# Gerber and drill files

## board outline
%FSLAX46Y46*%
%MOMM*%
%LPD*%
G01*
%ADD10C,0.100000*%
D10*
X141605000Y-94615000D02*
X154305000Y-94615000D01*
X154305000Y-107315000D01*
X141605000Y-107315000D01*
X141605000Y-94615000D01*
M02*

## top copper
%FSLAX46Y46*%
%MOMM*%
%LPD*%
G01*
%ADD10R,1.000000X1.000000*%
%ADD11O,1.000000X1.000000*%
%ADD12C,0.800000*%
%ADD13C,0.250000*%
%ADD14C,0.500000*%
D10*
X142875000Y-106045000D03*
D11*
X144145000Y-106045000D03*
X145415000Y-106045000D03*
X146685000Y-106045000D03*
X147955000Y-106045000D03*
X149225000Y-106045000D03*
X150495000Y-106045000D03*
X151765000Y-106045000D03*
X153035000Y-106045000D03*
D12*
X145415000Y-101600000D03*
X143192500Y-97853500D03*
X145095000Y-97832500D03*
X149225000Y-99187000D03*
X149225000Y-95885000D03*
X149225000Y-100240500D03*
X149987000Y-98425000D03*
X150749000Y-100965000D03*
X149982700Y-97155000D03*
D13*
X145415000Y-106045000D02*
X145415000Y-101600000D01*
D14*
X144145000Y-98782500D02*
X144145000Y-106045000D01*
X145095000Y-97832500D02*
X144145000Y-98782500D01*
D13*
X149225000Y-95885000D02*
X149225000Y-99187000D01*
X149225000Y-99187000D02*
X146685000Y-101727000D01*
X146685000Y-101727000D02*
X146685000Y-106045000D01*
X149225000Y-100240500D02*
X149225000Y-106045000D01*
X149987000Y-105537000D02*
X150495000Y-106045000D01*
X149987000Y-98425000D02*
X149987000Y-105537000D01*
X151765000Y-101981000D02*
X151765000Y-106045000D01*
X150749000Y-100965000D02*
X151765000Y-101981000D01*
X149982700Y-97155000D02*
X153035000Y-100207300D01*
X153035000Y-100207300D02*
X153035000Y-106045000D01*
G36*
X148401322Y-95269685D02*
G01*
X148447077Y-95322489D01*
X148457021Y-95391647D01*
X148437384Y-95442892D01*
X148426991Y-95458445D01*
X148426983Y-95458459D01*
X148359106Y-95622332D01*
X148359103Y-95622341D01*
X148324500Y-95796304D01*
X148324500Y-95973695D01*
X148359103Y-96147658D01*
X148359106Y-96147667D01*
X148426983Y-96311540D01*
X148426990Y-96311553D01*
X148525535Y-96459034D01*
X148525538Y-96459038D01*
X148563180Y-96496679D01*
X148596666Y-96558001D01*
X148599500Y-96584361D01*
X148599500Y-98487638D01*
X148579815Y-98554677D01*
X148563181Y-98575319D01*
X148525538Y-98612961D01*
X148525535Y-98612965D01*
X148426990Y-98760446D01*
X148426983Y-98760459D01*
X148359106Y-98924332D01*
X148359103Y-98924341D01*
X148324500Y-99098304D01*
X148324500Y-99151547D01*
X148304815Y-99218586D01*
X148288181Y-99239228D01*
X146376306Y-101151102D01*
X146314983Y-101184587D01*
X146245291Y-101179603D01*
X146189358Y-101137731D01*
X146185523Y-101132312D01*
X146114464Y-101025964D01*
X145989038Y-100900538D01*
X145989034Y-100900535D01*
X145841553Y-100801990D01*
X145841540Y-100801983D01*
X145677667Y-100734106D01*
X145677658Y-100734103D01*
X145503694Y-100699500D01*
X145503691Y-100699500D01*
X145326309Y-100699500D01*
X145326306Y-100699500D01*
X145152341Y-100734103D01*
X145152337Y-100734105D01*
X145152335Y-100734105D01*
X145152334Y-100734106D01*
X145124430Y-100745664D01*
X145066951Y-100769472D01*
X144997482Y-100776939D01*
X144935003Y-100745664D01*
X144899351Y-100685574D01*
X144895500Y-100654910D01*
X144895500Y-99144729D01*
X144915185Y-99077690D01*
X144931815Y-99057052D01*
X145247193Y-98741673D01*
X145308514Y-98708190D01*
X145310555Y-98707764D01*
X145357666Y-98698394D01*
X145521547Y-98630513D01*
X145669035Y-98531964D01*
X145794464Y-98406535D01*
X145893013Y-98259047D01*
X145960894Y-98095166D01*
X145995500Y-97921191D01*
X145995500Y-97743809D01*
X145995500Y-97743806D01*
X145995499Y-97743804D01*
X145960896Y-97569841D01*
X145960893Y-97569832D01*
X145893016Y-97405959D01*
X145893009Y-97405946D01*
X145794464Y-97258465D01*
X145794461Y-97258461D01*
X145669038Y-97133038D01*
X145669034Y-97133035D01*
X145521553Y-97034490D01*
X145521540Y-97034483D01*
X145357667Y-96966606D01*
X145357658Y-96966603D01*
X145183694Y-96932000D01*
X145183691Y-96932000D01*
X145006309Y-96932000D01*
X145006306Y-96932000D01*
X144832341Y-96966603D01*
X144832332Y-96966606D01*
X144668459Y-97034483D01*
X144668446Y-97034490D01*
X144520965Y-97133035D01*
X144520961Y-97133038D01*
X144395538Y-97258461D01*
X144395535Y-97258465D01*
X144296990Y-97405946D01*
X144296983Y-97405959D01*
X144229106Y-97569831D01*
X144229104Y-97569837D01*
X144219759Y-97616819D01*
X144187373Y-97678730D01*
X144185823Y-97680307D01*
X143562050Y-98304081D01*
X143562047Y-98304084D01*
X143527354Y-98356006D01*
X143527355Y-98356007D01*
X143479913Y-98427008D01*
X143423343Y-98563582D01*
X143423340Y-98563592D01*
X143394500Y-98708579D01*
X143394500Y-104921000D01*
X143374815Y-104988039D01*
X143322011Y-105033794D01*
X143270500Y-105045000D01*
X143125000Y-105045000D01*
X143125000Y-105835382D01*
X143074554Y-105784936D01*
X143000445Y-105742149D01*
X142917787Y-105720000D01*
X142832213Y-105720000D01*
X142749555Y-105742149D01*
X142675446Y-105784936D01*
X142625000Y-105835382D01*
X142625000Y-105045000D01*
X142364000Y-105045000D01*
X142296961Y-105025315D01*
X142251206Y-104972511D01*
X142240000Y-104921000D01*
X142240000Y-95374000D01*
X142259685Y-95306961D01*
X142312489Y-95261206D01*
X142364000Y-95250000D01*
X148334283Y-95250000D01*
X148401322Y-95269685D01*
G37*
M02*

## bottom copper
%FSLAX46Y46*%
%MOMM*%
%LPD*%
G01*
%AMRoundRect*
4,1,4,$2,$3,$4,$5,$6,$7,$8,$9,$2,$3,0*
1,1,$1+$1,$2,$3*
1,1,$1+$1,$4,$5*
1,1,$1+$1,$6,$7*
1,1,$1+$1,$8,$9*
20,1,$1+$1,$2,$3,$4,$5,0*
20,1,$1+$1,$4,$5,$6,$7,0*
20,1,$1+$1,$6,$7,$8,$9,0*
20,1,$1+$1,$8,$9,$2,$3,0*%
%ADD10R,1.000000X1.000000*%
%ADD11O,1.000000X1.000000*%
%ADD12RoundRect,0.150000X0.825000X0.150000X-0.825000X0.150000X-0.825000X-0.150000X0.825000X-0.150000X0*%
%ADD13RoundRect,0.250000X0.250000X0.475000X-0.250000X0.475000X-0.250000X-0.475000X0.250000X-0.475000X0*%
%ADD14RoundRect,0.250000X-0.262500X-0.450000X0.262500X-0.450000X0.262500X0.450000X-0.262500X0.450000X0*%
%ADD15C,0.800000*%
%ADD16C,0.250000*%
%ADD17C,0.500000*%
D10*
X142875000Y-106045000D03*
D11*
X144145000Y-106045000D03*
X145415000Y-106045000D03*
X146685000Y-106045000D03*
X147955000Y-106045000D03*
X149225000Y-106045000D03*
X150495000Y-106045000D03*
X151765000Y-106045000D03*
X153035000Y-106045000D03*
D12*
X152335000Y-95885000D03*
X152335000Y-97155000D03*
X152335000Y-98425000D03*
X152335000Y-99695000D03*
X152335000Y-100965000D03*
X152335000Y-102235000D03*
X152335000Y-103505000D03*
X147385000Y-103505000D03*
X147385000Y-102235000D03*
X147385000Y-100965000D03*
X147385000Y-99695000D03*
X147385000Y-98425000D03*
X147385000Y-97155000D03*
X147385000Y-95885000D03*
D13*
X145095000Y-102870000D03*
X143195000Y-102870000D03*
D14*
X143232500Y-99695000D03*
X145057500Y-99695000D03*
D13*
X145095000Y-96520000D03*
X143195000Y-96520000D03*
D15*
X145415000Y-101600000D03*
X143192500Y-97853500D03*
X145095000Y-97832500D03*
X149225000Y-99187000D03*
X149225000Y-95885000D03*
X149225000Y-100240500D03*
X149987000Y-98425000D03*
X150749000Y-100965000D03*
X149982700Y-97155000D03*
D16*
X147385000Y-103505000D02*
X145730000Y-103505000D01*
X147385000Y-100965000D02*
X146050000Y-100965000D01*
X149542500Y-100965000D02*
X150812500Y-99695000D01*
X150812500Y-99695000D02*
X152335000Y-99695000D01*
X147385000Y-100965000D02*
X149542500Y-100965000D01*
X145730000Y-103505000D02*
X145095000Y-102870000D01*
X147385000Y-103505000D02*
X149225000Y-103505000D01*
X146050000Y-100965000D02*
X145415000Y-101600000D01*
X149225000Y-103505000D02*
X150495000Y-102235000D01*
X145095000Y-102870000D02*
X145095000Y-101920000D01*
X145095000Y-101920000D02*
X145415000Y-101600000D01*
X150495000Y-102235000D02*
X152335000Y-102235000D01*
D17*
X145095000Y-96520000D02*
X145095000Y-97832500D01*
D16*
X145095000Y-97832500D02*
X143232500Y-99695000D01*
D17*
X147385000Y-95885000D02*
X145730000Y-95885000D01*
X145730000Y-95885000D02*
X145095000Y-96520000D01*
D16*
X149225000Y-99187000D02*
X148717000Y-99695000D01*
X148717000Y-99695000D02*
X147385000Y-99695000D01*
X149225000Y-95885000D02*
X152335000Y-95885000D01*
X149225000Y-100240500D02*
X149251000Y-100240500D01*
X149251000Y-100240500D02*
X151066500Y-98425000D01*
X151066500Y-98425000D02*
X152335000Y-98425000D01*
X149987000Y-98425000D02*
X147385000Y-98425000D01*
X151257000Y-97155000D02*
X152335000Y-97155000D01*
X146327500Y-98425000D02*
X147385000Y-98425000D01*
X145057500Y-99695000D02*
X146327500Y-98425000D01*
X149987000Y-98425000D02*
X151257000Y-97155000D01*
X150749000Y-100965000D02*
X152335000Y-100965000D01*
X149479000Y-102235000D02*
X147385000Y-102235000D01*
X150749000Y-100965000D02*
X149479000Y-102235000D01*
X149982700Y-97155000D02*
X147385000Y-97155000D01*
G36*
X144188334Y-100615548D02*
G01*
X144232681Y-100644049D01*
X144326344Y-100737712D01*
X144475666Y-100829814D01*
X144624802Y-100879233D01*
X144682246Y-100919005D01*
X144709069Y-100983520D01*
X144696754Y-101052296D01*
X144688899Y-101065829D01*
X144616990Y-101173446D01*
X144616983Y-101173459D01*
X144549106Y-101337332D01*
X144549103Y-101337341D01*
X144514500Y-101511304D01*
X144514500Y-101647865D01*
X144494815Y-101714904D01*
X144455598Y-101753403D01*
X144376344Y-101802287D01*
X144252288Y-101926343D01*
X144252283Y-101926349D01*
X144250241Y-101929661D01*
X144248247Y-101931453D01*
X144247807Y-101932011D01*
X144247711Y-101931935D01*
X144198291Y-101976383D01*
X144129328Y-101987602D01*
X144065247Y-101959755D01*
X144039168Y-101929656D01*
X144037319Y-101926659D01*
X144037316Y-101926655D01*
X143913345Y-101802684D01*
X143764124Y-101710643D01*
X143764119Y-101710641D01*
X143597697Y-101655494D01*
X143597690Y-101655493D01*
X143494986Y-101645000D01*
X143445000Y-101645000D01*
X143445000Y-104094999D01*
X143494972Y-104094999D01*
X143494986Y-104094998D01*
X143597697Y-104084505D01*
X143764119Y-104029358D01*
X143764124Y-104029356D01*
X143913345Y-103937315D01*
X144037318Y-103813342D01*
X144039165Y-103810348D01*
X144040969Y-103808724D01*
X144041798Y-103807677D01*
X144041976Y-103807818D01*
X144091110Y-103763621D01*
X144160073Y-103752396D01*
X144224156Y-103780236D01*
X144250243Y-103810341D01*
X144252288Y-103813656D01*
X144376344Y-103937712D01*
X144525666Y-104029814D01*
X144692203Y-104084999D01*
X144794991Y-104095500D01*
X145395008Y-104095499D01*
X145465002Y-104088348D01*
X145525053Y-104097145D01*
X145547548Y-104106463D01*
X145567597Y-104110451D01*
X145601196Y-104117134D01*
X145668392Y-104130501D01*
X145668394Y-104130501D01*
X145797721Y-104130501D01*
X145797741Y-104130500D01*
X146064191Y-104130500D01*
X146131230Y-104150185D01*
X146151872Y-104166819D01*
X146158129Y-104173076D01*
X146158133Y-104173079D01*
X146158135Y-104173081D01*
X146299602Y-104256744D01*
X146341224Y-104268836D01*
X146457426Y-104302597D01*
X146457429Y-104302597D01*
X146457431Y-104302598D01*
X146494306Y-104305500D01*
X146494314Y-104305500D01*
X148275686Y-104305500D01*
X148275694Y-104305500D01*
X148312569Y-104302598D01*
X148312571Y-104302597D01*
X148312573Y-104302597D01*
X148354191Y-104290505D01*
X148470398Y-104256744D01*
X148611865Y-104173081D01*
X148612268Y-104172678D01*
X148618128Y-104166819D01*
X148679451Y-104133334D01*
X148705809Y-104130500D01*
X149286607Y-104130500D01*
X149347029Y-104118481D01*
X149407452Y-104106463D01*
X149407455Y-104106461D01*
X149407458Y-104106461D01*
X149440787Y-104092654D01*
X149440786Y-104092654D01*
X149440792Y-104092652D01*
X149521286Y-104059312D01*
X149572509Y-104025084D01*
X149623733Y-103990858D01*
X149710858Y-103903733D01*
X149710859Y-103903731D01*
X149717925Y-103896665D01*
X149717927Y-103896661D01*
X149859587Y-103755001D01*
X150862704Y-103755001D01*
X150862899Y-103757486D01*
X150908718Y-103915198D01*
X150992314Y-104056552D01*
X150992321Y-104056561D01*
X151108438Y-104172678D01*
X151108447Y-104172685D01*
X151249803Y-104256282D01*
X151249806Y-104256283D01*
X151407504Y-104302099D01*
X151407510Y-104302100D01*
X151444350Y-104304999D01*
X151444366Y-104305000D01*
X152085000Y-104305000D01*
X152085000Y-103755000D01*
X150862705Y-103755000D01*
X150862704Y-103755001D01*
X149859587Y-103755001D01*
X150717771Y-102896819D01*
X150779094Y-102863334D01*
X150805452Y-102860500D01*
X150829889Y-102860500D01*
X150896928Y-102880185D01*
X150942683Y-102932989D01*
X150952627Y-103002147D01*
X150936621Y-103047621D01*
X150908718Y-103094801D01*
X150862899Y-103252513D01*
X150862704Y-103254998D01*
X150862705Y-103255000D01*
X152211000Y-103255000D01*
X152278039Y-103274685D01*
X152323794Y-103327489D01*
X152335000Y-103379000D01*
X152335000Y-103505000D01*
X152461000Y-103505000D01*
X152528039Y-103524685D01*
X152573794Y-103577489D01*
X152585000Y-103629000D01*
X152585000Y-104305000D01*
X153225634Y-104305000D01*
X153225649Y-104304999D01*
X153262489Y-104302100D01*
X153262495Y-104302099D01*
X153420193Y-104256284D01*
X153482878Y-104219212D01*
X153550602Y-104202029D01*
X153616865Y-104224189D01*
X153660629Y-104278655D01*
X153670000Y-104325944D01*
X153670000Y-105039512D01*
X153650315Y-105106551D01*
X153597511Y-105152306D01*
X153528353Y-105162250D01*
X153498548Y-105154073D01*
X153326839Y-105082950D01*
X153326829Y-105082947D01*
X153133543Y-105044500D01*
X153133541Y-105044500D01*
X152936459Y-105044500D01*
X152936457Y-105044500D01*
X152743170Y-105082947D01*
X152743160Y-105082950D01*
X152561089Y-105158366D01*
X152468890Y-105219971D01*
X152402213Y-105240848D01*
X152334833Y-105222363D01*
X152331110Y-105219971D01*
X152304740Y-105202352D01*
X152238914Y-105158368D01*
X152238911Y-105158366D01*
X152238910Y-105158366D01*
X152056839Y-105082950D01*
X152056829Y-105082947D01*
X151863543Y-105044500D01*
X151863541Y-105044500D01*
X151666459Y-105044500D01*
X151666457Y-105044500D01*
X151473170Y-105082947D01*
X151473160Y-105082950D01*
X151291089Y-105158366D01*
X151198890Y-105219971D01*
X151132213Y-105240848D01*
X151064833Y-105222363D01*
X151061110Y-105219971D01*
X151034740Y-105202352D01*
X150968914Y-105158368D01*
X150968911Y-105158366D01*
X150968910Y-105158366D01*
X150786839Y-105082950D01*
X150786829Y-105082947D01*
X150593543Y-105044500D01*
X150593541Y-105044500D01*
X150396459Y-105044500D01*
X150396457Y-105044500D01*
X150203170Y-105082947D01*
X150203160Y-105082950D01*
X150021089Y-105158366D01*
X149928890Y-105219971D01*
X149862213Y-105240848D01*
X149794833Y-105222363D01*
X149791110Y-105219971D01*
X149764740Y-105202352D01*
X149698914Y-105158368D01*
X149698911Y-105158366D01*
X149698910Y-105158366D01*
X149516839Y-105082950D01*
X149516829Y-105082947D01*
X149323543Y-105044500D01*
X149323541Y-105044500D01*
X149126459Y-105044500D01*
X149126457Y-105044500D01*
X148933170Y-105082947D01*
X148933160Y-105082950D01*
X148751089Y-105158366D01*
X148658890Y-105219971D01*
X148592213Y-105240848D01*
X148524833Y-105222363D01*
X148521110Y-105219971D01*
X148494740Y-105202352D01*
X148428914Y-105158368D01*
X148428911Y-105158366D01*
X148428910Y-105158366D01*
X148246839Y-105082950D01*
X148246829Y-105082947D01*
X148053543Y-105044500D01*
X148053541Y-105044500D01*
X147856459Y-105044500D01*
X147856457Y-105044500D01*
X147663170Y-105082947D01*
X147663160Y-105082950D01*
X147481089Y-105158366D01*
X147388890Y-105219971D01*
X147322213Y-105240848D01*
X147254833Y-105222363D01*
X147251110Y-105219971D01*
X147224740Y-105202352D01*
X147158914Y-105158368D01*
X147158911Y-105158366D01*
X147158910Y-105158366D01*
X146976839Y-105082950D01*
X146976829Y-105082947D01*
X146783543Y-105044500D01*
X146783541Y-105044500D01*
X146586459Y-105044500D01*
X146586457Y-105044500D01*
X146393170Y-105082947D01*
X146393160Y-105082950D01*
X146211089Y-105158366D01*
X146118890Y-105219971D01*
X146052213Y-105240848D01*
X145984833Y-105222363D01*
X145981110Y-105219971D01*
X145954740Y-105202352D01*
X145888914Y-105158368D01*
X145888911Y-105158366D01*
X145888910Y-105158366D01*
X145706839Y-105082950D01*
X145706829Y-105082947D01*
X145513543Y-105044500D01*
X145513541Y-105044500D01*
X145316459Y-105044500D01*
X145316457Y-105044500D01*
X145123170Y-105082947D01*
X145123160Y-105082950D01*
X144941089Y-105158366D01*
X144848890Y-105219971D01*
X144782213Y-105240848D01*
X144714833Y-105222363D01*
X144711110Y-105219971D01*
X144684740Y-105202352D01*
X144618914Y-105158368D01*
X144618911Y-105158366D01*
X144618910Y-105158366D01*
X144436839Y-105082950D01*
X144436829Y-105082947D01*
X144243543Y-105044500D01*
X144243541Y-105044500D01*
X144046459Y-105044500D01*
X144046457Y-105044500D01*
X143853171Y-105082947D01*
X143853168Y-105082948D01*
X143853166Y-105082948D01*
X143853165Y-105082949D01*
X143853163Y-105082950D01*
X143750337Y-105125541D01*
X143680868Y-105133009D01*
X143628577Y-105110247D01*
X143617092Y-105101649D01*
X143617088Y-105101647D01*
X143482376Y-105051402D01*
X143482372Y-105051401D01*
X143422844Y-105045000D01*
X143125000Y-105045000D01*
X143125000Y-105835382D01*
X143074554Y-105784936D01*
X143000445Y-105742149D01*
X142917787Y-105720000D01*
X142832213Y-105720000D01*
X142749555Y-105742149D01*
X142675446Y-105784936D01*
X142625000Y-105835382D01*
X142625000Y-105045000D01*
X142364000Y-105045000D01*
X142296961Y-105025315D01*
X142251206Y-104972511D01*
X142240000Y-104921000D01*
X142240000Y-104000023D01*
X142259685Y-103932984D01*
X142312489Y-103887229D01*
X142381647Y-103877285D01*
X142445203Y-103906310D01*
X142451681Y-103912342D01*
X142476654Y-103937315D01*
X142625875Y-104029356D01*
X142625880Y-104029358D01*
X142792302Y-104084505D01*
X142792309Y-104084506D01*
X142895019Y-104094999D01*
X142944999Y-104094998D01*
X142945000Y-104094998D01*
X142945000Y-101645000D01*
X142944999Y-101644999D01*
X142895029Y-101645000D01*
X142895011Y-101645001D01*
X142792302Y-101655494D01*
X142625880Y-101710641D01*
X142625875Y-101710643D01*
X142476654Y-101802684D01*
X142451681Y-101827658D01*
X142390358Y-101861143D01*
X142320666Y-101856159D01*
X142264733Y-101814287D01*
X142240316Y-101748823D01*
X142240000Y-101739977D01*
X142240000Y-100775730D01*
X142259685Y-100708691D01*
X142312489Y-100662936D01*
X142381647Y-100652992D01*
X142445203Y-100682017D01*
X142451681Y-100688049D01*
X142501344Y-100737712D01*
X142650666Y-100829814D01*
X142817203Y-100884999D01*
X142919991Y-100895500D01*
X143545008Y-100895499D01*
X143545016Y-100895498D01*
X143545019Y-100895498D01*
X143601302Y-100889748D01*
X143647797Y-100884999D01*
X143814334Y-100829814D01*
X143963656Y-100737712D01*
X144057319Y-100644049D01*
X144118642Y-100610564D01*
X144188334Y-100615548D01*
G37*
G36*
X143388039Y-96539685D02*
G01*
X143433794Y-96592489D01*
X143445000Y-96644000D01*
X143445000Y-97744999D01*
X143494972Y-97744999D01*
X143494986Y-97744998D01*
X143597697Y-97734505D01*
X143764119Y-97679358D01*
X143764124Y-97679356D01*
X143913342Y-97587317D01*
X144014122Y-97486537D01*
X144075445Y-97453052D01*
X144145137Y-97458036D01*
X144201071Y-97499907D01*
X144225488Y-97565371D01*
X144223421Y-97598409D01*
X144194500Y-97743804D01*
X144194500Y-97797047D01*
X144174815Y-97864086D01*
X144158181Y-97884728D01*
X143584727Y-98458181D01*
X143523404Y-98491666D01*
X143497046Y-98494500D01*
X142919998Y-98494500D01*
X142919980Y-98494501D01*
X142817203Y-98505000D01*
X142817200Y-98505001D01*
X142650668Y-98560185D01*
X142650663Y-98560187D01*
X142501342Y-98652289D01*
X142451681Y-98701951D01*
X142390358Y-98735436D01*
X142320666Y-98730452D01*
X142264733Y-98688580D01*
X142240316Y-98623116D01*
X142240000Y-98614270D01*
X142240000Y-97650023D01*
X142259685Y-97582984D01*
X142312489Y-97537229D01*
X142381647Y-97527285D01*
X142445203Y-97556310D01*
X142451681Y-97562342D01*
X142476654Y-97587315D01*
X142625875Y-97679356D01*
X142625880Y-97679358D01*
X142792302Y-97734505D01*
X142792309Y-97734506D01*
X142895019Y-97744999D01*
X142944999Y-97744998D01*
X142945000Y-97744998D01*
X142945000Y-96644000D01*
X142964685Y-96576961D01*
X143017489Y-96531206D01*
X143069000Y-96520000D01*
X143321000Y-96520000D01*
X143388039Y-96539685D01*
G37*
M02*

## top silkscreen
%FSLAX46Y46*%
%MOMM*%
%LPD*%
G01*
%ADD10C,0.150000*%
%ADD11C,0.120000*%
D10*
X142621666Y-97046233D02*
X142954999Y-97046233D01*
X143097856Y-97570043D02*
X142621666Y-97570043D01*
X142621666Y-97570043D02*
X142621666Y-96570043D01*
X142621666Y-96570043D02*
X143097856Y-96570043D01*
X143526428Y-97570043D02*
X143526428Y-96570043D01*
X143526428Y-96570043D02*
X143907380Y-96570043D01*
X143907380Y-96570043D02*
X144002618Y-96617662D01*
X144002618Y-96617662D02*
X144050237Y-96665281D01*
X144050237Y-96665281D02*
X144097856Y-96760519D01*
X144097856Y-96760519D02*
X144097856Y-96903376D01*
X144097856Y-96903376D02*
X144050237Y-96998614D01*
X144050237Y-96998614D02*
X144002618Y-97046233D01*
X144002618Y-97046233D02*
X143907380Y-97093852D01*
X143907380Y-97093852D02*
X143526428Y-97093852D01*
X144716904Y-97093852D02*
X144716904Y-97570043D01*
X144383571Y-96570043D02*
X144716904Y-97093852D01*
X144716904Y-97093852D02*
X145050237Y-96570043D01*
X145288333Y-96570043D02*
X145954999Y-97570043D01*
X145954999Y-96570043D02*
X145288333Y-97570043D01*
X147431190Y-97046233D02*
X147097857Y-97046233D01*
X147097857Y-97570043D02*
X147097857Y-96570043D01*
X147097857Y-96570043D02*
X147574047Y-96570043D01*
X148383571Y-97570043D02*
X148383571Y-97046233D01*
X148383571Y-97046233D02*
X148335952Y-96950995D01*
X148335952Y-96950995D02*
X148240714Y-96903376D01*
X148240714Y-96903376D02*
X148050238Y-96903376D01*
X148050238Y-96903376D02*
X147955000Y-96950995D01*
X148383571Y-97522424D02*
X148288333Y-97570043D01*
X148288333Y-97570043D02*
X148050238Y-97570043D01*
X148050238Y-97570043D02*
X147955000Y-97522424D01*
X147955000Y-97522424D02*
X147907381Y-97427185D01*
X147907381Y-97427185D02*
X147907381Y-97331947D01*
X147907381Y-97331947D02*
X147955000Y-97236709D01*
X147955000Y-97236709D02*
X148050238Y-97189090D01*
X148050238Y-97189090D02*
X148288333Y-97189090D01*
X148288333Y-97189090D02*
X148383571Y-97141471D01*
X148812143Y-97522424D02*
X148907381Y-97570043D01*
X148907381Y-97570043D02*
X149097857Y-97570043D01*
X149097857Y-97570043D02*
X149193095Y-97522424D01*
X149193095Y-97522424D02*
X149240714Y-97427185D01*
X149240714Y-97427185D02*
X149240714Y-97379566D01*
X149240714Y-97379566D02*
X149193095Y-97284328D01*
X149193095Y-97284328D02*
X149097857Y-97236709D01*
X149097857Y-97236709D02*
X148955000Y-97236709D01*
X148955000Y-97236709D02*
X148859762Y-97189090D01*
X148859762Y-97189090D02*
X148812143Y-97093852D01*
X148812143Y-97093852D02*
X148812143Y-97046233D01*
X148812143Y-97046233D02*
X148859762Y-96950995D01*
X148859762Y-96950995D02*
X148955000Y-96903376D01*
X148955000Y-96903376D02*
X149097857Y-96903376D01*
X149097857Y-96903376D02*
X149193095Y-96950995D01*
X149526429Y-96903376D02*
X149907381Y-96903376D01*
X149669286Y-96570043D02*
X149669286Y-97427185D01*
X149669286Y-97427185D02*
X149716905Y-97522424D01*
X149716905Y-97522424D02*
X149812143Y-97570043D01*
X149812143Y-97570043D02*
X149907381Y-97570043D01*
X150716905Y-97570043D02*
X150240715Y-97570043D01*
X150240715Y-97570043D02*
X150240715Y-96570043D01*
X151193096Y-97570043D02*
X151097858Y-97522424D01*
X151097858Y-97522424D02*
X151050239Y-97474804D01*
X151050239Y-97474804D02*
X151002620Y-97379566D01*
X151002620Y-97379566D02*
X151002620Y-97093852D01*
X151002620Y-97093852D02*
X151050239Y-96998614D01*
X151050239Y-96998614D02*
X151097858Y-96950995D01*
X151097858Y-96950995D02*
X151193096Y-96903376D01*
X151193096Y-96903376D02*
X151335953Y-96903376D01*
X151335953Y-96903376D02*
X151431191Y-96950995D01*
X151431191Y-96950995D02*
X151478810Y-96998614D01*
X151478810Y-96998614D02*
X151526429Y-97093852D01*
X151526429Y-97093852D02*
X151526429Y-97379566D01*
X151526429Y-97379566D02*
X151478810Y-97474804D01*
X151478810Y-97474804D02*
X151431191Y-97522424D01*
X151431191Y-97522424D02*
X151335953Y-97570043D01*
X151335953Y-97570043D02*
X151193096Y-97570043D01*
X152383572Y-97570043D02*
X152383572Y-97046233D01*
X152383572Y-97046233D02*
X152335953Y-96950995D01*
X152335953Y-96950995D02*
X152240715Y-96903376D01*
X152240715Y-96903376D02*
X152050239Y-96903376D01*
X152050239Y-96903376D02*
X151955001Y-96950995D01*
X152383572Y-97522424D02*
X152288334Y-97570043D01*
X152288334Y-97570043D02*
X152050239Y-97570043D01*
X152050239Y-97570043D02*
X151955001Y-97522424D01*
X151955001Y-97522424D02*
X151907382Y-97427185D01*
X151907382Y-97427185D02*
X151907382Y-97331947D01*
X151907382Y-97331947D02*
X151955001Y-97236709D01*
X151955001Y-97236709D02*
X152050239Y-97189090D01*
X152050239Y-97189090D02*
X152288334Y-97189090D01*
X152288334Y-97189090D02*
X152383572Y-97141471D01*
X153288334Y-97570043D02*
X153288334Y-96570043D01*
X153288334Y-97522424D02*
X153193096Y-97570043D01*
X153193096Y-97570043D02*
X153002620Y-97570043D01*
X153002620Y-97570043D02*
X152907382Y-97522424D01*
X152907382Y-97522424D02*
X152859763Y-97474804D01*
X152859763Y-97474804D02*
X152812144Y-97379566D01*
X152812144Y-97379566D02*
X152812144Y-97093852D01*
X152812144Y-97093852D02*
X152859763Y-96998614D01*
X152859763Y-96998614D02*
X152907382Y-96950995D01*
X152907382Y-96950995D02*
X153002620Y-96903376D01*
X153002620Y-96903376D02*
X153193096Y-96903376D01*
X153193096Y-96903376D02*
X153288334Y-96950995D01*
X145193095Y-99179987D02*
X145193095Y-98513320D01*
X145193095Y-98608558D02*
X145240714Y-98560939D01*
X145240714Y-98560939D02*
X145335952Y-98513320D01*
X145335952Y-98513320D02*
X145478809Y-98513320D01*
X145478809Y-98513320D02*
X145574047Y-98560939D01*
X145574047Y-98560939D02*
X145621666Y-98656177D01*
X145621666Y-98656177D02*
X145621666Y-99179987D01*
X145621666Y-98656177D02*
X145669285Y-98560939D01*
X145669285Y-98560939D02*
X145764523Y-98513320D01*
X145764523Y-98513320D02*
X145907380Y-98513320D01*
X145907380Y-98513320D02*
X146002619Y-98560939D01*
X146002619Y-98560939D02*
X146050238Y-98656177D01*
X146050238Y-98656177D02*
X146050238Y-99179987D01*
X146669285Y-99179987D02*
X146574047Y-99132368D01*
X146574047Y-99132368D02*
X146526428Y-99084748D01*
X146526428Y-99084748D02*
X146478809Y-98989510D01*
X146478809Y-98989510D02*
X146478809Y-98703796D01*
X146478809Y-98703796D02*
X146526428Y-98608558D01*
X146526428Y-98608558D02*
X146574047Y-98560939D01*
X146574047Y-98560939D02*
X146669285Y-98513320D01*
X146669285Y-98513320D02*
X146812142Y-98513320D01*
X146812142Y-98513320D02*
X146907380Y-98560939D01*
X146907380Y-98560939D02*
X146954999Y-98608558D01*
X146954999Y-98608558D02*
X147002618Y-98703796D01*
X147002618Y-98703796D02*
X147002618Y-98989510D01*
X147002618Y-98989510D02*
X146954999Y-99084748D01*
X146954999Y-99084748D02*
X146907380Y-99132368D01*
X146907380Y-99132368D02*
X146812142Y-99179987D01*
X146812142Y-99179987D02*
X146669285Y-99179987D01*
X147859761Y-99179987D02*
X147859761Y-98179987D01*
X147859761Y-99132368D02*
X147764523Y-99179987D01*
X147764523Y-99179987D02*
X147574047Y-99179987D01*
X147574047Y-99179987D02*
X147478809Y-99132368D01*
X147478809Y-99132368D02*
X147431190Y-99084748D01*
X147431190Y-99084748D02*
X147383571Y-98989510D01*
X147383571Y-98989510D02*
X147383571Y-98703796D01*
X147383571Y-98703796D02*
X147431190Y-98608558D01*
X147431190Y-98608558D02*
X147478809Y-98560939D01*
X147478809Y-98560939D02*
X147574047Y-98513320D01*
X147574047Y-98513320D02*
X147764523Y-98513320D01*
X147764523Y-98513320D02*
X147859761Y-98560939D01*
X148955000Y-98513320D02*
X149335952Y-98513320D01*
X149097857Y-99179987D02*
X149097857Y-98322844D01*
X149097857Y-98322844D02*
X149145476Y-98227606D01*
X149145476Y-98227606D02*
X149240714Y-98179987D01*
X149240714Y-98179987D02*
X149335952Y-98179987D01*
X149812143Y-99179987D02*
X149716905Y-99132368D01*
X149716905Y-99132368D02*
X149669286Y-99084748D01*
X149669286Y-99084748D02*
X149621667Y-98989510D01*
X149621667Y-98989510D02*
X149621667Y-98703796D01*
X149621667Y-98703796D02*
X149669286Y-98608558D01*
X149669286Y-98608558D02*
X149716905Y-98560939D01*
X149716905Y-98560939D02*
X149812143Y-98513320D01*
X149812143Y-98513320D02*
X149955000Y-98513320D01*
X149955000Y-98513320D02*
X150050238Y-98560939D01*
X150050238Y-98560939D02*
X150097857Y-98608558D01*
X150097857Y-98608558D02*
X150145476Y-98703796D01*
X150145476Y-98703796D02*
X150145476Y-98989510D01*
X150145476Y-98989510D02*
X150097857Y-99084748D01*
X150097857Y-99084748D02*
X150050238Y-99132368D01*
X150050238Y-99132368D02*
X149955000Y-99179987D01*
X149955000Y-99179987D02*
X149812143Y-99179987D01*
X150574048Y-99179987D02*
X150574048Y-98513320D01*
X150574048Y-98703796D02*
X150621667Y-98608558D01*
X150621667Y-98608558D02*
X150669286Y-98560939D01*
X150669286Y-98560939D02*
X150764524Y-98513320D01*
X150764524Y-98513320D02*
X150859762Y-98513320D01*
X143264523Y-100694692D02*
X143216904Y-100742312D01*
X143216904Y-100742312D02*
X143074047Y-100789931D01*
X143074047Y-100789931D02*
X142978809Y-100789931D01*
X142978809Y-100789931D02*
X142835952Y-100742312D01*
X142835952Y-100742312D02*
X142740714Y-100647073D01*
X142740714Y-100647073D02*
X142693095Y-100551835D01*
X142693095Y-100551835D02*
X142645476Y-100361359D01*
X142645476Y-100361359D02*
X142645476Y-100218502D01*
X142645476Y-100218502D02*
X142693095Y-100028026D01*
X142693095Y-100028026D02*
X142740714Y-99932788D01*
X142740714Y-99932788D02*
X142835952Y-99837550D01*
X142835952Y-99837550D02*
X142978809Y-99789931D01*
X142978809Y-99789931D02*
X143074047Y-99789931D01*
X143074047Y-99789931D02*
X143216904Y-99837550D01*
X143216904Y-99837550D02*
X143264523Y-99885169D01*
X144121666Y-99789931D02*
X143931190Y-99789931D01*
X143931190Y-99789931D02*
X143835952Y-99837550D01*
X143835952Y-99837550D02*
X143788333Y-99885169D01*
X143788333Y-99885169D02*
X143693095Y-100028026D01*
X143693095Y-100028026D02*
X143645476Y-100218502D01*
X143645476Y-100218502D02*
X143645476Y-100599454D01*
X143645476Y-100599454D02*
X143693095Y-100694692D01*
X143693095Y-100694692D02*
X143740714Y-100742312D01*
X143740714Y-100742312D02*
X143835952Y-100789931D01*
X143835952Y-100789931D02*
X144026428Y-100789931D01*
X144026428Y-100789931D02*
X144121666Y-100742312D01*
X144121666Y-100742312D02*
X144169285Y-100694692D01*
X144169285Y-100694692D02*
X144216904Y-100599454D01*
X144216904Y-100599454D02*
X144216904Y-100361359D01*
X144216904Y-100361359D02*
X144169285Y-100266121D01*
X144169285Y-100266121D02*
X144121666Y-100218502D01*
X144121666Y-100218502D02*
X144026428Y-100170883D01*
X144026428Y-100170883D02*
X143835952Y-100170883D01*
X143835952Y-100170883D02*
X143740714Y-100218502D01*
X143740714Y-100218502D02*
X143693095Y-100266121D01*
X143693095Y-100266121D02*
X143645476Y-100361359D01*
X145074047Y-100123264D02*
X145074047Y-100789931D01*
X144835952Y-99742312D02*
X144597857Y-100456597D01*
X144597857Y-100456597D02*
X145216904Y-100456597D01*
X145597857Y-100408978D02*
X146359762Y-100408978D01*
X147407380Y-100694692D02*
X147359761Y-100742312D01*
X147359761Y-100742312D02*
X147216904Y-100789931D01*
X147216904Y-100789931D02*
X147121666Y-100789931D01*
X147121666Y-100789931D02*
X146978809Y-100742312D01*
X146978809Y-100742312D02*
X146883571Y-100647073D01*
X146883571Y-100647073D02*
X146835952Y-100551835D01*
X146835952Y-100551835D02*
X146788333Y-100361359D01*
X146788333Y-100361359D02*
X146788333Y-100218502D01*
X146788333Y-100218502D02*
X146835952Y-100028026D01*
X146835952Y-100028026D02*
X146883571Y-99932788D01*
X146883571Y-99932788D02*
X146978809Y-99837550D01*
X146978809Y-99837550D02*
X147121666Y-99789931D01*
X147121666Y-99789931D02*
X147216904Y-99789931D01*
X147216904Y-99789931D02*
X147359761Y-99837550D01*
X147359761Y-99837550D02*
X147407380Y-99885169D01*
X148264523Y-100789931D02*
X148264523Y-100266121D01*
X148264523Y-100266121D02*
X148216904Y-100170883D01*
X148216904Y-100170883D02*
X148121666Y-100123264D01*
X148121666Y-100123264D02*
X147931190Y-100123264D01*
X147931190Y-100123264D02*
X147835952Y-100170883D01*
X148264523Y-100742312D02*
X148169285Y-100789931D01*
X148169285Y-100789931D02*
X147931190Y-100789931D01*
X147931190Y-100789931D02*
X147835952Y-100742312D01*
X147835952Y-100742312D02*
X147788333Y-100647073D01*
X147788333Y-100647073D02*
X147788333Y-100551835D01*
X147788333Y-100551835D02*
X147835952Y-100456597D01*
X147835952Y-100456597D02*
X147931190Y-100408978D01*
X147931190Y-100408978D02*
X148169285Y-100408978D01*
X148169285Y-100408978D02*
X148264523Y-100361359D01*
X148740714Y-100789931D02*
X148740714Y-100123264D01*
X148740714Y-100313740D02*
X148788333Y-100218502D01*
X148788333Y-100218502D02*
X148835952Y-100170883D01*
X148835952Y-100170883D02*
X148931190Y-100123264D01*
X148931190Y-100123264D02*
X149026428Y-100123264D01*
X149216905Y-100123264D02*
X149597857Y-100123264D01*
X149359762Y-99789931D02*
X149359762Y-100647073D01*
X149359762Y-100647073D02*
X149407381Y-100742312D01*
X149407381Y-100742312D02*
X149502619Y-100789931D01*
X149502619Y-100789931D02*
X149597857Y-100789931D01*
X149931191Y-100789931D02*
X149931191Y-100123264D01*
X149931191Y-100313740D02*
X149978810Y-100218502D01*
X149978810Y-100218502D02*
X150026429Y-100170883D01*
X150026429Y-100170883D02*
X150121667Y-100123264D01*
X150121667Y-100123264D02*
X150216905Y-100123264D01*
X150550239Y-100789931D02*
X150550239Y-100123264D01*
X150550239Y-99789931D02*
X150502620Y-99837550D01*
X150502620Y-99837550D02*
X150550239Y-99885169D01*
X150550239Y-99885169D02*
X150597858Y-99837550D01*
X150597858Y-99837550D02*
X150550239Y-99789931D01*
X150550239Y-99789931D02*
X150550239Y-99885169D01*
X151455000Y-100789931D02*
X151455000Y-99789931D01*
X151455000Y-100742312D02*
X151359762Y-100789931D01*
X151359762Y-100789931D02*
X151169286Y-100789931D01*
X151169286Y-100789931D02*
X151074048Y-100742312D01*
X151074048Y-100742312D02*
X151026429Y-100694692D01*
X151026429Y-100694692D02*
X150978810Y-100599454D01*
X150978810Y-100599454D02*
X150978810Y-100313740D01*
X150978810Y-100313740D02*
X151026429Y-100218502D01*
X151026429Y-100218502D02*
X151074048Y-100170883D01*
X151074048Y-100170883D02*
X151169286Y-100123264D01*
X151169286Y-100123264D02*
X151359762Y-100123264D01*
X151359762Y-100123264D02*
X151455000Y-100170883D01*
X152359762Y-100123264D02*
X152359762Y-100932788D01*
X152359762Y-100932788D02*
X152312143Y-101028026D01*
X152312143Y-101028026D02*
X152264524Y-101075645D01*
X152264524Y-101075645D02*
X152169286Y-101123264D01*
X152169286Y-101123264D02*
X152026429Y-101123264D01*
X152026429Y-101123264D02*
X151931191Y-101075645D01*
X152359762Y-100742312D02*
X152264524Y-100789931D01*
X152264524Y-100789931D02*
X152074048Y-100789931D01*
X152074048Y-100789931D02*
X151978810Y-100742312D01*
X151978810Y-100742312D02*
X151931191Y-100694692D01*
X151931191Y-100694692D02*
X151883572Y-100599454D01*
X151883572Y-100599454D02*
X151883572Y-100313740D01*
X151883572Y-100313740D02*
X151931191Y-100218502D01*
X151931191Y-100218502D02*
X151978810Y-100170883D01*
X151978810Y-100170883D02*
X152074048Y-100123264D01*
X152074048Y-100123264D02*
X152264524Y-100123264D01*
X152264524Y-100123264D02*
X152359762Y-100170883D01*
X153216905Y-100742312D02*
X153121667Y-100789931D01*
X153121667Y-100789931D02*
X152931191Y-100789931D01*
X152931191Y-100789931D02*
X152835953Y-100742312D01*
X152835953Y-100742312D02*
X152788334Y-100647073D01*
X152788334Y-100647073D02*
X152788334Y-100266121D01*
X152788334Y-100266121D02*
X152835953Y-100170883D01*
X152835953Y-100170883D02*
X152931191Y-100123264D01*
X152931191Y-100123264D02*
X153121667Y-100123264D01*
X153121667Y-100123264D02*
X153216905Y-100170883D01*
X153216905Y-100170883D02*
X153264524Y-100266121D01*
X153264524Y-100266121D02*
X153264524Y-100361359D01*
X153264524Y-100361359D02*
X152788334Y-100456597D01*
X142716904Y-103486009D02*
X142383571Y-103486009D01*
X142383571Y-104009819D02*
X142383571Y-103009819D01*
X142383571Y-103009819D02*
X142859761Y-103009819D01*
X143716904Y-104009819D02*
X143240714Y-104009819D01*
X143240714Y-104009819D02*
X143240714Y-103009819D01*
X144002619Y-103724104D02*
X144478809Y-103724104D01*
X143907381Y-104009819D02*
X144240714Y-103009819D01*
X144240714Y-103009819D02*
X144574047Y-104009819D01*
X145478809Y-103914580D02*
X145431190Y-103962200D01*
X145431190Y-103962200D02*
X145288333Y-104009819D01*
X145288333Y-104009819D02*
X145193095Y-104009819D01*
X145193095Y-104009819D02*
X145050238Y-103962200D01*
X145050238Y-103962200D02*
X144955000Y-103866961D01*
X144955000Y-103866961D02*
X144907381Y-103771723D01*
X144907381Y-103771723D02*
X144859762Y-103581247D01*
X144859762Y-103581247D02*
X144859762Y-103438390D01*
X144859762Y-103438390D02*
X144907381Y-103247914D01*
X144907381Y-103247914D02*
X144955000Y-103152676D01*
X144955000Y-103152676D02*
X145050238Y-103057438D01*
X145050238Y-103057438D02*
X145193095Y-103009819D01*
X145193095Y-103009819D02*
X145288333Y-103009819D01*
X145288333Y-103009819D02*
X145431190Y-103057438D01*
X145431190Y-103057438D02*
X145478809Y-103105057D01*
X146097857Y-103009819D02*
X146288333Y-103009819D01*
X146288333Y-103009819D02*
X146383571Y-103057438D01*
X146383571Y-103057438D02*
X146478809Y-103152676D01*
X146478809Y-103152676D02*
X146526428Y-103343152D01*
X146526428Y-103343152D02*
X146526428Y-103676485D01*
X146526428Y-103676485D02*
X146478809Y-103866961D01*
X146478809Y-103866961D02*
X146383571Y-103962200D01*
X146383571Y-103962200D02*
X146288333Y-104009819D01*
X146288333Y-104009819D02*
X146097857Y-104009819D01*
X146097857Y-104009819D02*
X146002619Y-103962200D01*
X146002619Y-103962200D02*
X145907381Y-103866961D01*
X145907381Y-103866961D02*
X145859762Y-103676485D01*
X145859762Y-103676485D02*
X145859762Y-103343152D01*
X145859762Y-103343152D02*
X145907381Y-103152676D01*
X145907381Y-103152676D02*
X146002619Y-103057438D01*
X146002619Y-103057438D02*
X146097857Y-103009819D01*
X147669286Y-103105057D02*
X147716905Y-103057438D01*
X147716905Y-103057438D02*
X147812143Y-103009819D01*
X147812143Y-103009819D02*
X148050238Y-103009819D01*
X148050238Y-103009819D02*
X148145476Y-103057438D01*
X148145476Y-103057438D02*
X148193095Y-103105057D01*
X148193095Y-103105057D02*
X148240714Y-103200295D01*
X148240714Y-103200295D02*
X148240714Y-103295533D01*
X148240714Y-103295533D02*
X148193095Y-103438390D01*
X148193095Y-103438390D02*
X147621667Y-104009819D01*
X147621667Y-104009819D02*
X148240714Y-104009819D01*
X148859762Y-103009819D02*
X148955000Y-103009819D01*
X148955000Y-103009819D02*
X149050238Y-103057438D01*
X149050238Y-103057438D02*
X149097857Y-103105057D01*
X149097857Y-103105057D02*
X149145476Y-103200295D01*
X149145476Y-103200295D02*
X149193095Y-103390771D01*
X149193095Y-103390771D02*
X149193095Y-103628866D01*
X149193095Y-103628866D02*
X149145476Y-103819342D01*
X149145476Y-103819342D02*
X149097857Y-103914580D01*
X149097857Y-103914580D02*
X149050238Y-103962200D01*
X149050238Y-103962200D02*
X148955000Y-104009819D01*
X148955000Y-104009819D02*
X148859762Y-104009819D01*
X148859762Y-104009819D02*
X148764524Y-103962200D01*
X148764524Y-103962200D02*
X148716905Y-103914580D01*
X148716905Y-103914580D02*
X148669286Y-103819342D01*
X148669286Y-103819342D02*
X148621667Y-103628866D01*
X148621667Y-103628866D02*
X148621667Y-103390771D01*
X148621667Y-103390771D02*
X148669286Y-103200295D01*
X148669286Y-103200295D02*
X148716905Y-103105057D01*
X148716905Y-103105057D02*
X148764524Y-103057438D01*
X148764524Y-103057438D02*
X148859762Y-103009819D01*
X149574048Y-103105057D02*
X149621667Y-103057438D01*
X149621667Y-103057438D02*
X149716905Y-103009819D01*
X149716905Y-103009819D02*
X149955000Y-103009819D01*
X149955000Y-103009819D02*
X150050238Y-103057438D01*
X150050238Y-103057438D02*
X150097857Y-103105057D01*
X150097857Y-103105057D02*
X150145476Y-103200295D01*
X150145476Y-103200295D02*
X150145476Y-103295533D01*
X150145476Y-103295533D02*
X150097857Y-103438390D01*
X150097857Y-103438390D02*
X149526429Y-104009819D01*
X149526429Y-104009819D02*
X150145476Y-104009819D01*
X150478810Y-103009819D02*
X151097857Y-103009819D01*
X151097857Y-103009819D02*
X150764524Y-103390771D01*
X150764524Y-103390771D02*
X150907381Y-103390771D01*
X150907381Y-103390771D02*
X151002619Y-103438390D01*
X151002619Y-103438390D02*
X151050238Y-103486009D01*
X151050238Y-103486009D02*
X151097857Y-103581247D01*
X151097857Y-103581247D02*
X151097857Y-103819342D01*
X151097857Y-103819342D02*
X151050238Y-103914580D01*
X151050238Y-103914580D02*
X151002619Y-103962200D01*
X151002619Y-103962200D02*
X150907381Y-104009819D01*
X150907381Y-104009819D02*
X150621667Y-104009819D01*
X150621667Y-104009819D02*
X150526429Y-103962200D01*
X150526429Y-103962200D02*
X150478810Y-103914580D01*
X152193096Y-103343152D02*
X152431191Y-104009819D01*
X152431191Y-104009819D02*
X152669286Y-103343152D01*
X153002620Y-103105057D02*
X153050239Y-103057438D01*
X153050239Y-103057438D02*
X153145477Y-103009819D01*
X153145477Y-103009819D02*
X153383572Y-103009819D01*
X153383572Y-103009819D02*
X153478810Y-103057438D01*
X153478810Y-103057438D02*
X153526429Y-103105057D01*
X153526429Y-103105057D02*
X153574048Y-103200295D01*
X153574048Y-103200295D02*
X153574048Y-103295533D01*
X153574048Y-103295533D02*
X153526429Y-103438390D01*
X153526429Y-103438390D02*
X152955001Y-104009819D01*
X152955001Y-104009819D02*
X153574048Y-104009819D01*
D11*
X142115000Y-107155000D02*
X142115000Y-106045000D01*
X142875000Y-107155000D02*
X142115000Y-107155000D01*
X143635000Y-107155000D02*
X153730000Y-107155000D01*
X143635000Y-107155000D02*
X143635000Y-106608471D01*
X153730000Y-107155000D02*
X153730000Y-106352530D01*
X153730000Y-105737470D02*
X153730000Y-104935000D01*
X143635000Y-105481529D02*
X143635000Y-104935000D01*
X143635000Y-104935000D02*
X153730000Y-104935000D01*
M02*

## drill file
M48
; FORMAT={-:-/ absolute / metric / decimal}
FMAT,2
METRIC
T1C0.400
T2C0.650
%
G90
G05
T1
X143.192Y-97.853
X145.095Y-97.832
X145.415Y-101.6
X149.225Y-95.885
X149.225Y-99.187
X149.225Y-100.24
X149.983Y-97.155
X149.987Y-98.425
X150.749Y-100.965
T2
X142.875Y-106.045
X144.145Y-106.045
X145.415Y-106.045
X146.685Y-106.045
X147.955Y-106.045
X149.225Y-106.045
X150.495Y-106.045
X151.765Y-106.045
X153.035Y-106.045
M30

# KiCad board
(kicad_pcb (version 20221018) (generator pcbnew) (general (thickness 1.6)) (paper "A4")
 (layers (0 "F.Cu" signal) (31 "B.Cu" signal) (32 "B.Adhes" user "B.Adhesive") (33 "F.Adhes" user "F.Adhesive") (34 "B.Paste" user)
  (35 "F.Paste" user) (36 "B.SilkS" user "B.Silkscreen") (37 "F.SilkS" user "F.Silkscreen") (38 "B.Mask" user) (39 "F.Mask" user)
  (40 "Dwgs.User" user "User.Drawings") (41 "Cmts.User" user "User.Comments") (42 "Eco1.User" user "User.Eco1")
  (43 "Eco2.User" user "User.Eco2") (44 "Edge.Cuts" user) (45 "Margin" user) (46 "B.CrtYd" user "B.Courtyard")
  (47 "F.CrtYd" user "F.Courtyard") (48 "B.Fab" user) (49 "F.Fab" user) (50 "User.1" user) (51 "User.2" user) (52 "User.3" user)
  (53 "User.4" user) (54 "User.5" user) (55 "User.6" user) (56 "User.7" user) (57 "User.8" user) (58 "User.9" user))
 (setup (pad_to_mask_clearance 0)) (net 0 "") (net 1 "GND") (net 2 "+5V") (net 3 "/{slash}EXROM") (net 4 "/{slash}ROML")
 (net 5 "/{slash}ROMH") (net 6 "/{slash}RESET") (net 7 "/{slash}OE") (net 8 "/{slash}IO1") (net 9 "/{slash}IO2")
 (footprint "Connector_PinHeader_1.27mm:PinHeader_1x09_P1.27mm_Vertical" (layer "F.Cu") (at 142.875 106.045 90)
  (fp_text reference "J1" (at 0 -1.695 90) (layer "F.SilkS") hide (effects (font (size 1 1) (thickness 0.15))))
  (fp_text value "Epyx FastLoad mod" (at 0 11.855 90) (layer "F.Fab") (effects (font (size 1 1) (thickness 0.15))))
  (fp_line (start -1.11 -0.76) (end 0 -0.76) (stroke (width 0.12) (type solid)) (layer "F.SilkS"))
  (fp_line (start -1.11 0) (end -1.11 -0.76) (stroke (width 0.12) (type solid)) (layer "F.SilkS"))
  (fp_line (start -1.11 0.76) (end -1.11 10.855) (stroke (width 0.12) (type solid)) (layer "F.SilkS"))
  (fp_line (start -1.11 0.76) (end -0.563471 0.76) (stroke (width 0.12) (type solid)) (layer "F.SilkS"))
  (fp_line (start -1.11 10.855) (end -0.30753 10.855) (stroke (width 0.12) (type solid)) (layer "F.SilkS"))
  (fp_line (start 0.30753 10.855) (end 1.11 10.855) (stroke (width 0.12) (type solid)) (layer "F.SilkS"))
  (fp_line (start 0.563471 0.76) (end 1.11 0.76) (stroke (width 0.12) (type solid)) (layer "F.SilkS"))
  (fp_line (start 1.11 0.76) (end 1.11 10.855) (stroke (width 0.12) (type solid)) (layer "F.SilkS"))
  (pad "1" thru_hole rect (at 0 0 90) (size 1 1) (drill 0.65) (layers "*.Cu" "*.Mask") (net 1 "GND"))
  (pad "2" thru_hole oval (at 0 1.27 90) (size 1 1) (drill 0.65) (layers "*.Cu" "*.Mask") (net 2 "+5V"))
  (pad "3" thru_hole oval (at 0 2.54 90) (size 1 1) (drill 0.65) (layers "*.Cu" "*.Mask") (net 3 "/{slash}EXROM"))
  (pad "4" thru_hole oval (at 0 3.81 90) (size 1 1) (drill 0.65) (layers "*.Cu" "*.Mask") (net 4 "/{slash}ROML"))
  (pad "5" thru_hole oval (at 0 5.08 90) (size 1 1) (drill 0.65) (layers "*.Cu" "*.Mask") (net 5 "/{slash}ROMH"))
  (pad "6" thru_hole oval (at 0 6.35 90) (size 1 1) (drill 0.65) (layers "*.Cu" "*.Mask") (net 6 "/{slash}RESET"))
  (pad "7" thru_hole oval (at 0 7.62 90) (size 1 1) (drill 0.65) (layers "*.Cu" "*.Mask") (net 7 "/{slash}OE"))
  (pad "8" thru_hole oval (at 0 8.89 90) (size 1 1) (drill 0.65) (layers "*.Cu" "*.Mask") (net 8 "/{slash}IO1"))
  (pad "9" thru_hole oval (at 0 10.16 90) (size 1 1) (drill 0.65) (layers "*.Cu" "*.Mask") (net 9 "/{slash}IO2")))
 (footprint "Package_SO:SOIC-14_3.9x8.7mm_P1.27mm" (layer "B.Cu") (at 149.86 99.695 180)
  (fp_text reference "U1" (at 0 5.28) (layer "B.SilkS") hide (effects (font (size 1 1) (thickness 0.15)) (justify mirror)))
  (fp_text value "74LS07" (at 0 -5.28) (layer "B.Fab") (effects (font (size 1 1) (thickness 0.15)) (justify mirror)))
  (pad "1" smd roundrect (at -2.475 3.81 180) (size 1.95 0.6) (layers "B.Cu" "B.Paste" "B.Mask") (roundrect_rratio 0.25)
   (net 4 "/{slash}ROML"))
  (pad "2" smd roundrect (at -2.475 2.54 180) (size 1.95 0.6) (layers "B.Cu" "B.Paste" "B.Mask") (roundrect_rratio 0.25)
   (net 7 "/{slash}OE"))
  (pad "3" smd roundrect (at -2.475 1.27 180) (size 1.95 0.6) (layers "B.Cu" "B.Paste" "B.Mask") (roundrect_rratio 0.25)
   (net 6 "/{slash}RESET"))
  (pad "4" smd roundrect (at -2.475 0 180) (size 1.95 0.6) (layers "B.Cu" "B.Paste" "B.Mask") (roundrect_rratio 0.25)
   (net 3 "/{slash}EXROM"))
  (pad "5" smd roundrect (at -2.475 -1.27 180) (size 1.95 0.6) (layers "B.Cu" "B.Paste" "B.Mask") (roundrect_rratio 0.25)
   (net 8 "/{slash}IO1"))
  (pad "6" smd roundrect (at -2.475 -2.54 180) (size 1.95 0.6) (layers "B.Cu" "B.Paste" "B.Mask") (roundrect_rratio 0.25)
   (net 3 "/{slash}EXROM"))
  (pad "7" smd roundrect (at -2.475 -3.81 180) (size 1.95 0.6) (layers "B.Cu" "B.Paste" "B.Mask") (roundrect_rratio 0.25) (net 1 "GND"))
  (pad "8" smd roundrect (at 2.475 -3.81 180) (size 1.95 0.6) (layers "B.Cu" "B.Paste" "B.Mask") (roundrect_rratio 0.25)
   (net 3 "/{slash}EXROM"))
  (pad "9" smd roundrect (at 2.475 -2.54 180) (size 1.95 0.6) (layers "B.Cu" "B.Paste" "B.Mask") (roundrect_rratio 0.25)
   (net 8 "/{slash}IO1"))
  (pad "10" smd roundrect (at 2.475 -1.27 180) (size 1.95 0.6) (layers "B.Cu" "B.Paste" "B.Mask") (roundrect_rratio 0.25)
   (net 3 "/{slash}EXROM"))
  (pad "11" smd roundrect (at 2.475 0 180) (size 1.95 0.6) (layers "B.Cu" "B.Paste" "B.Mask") (roundrect_rratio 0.25) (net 4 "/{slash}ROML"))
  (pad "12" smd roundrect (at 2.475 1.27 180) (size 1.95 0.6) (layers "B.Cu" "B.Paste" "B.Mask") (roundrect_rratio 0.25)
   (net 7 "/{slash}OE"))
  (pad "13" smd roundrect (at 2.475 2.54 180) (size 1.95 0.6) (layers "B.Cu" "B.Paste" "B.Mask") (roundrect_rratio 0.25)
   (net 9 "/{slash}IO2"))
  (pad "14" smd roundrect (at 2.475 3.81 180) (size 1.95 0.6) (layers "B.Cu" "B.Paste" "B.Mask") (roundrect_rratio 0.25) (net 2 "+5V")))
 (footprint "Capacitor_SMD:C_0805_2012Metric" (layer "B.Cu") (at 144.145 102.87 180)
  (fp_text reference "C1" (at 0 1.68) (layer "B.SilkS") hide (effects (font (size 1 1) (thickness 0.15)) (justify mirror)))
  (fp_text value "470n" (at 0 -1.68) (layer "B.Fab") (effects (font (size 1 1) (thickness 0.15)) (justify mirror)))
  (pad "1" smd roundrect (at -0.95 0 180) (size 1 1.45) (layers "B.Cu" "B.Paste" "B.Mask") (roundrect_rratio 0.25) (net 3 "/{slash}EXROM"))
  (pad "2" smd roundrect (at 0.95 0 180) (size 1 1.45) (layers "B.Cu" "B.Paste" "B.Mask") (roundrect_rratio 0.25) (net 1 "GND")))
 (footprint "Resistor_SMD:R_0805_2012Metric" (layer "B.Cu") (at 144.145 99.695)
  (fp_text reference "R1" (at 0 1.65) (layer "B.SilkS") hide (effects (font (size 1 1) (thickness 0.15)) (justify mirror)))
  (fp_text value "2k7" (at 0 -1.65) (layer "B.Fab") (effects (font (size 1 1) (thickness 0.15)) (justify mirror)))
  (pad "1" smd roundrect (at -0.9125 0) (size 1.025 1.4) (layers "B.Cu" "B.Paste" "B.Mask") (roundrect_rratio 0.243902) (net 2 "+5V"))
  (pad "2" smd roundrect (at 0.9125 0) (size 1.025 1.4) (layers "B.Cu" "B.Paste" "B.Mask") (roundrect_rratio 0.243902) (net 7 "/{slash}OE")))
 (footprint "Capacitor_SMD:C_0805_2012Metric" (layer "B.Cu") (at 144.145 96.52 180)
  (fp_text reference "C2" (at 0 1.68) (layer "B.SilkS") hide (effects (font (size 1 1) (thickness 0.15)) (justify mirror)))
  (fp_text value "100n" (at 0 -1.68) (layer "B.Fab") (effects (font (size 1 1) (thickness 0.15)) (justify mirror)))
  (pad "1" smd roundrect (at -0.95 0 180) (size 1 1.45) (layers "B.Cu" "B.Paste" "B.Mask") (roundrect_rratio 0.25) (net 2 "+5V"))
  (pad "2" smd roundrect (at 0.95 0 180) (size 1 1.45) (layers "B.Cu" "B.Paste" "B.Mask") (roundrect_rratio 0.25) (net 1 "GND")))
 (gr_rect (start 141.605 94.615) (end 154.305 107.315) (stroke (width 0.1) (type default)) (fill none) (layer "Edge.Cuts"))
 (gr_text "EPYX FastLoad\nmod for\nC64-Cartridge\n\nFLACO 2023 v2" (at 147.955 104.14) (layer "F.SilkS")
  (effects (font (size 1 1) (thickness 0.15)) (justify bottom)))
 (segment (start 145.415 106.045) (end 145.415 101.6) (width 0.25) (layer "F.Cu") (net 3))
 (via (at 145.415 101.6) (size 0.8) (drill 0.4) (layers "F.Cu" "B.Cu") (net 3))
 (segment (start 147.385 103.505) (end 145.73 103.505) (width 0.25) (layer "B.Cu") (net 3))
 (segment (start 147.385 100.965) (end 146.05 100.965) (width 0.25) (layer "B.Cu") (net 3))
 (segment (start 149.5425 100.965) (end 150.8125 99.695) (width 0.25) (layer "B.Cu") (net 3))
 (segment (start 150.8125 99.695) (end 152.335 99.695) (width 0.25) (layer "B.Cu") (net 3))
 (segment (start 147.385 100.965) (end 149.5425 100.965) (width 0.25) (layer "B.Cu") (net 3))
 (segment (start 145.73 103.505) (end 145.095 102.87) (width 0.25) (layer "B.Cu") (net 3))
 (segment (start 147.385 103.505) (end 149.225 103.505) (width 0.25) (layer "B.Cu") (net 3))
 (segment (start 146.05 100.965) (end 145.415 101.6) (width 0.25) (layer "B.Cu") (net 3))
 (segment (start 149.225 103.505) (end 150.495 102.235) (width 0.25) (layer "B.Cu") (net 3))
 (segment (start 145.095 102.87) (end 145.095 101.92) (width 0.25) (layer "B.Cu") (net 3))
 (segment (start 145.095 101.92) (end 145.415 101.6) (width 0.25) (layer "B.Cu") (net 3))
 (segment (start 150.495 102.235) (end 152.335 102.235) (width 0.25) (layer "B.Cu") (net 3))
 (via (at 143.1925 97.8535) (size 0.8) (drill 0.4) (layers "F.Cu" "B.Cu") (free) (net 1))
 (segment (start 144.145 98.7825) (end 144.145 106.045) (width 0.5) (layer "F.Cu") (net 2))
 (segment (start 145.095 97.8325) (end 144.145 98.7825) (width 0.5) (layer "F.Cu") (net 2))
 (via (at 145.095 97.8325) (size 0.8) (drill 0.4) (layers "F.Cu" "B.Cu") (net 2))
 (segment (start 145.095 96.52) (end 145.095 97.8325) (width 0.5) (layer "B.Cu") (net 2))
 (segment (start 145.095 97.8325) (end 143.2325 99.695) (width 0.25) (layer "B.Cu") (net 2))
 (segment (start 147.385 95.885) (end 145.73 95.885) (width 0.5) (layer "B.Cu") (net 2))
 (segment (start 145.73 95.885) (end 145.095 96.52) (width 0.5) (layer "B.Cu") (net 2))
 (segment (start 149.225 95.885) (end 149.225 99.187) (width 0.25) (layer "F.Cu") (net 4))
 (segment (start 149.225 99.187) (end 146.685 101.727) (width 0.25) (layer "F.Cu") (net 4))
 (segment (start 146.685 101.727) (end 146.685 106.045) (width 0.25) (layer "F.Cu") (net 4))
 (via (at 149.225 99.187) (size 0.8) (drill 0.4) (layers "F.Cu" "B.Cu") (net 4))
 (via (at 149.225 95.885) (size 0.8) (drill 0.4) (layers "F.Cu" "B.Cu") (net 4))
 (segment (start 149.225 99.187) (end 148.717 99.695) (width 0.25) (layer "B.Cu") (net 4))
 (segment (start 148.717 99.695) (end 147.385 99.695) (width 0.25) (layer "B.Cu") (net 4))
 (segment (start 149.225 95.885) (end 152.335 95.885) (width 0.25) (layer "B.Cu") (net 4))
 (segment (start 149.225 100.2405) (end 149.225 106.045) (width 0.25) (layer "F.Cu") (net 6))
 (via (at 149.225 100.2405) (size 0.8) (drill 0.4) (layers "F.Cu" "B.Cu") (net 6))
 (segment (start 149.225 100.2405) (end 149.251 100.2405) (width 0.25) (layer "B.Cu") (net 6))
 (segment (start 149.251 100.2405) (end 151.0665 98.425) (width 0.25) (layer "B.Cu") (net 6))
 (segment (start 151.0665 98.425) (end 152.335 98.425) (width 0.25) (layer "B.Cu") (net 6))
 (segment (start 149.987 105.537) (end 150.495 106.045) (width 0.25) (layer "F.Cu") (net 7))
 (segment (start 149.987 98.425) (end 149.987 105.537) (width 0.25) (layer "F.Cu") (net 7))
 (via (at 149.987 98.425) (size 0.8) (drill 0.4) (layers "F.Cu" "B.Cu") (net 7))
 (segment (start 149.987 98.425) (end 147.385 98.425) (width 0.25) (layer "B.Cu") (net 7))
 (segment (start 151.257 97.155) (end 152.335 97.155) (width 0.25) (layer "B.Cu") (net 7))
 (segment (start 146.3275 98.425) (end 147.385 98.425) (width 0.25) (layer "B.Cu") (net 7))
 (segment (start 145.0575 99.695) (end 146.3275 98.425) (width 0.25) (layer "B.Cu") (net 7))
 (segment (start 149.987 98.425) (end 151.257 97.155) (width 0.25) (layer "B.Cu") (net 7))
 (segment (start 151.765 101.981) (end 151.765 106.045) (width 0.25) (layer "F.Cu") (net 8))
 (segment (start 150.749 100.965) (end 151.765 101.981) (width 0.25) (layer "F.Cu") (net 8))
 (via (at 150.749 100.965) (size 0.8) (drill 0.4) (layers "F.Cu" "B.Cu") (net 8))
 (segment (start 150.749 100.965) (end 152.335 100.965) (width 0.25) (layer "B.Cu") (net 8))
 (segment (start 149.479 102.235) (end 147.385 102.235) (width 0.25) (layer "B.Cu") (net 8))
 (segment (start 150.749 100.965) (end 149.479 102.235) (width 0.25) (layer "B.Cu") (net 8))
 (segment (start 149.9827 97.155) (end 153.035 100.2073) (width 0.25) (layer "F.Cu") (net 9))
 (segment (start 153.035 100.2073) (end 153.035 106.045) (width 0.25) (layer "F.Cu") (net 9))
 (via (at 149.9827 97.155) (size 0.8) (drill 0.4) (layers "F.Cu" "B.Cu") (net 9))
 (segment (start 149.9827 97.155) (end 147.385 97.155) (width 0.25) (layer "B.Cu") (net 9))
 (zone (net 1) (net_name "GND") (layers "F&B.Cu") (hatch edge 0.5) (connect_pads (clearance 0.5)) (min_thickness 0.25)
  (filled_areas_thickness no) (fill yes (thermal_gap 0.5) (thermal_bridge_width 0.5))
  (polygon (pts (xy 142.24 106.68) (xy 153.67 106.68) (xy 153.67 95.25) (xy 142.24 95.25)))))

